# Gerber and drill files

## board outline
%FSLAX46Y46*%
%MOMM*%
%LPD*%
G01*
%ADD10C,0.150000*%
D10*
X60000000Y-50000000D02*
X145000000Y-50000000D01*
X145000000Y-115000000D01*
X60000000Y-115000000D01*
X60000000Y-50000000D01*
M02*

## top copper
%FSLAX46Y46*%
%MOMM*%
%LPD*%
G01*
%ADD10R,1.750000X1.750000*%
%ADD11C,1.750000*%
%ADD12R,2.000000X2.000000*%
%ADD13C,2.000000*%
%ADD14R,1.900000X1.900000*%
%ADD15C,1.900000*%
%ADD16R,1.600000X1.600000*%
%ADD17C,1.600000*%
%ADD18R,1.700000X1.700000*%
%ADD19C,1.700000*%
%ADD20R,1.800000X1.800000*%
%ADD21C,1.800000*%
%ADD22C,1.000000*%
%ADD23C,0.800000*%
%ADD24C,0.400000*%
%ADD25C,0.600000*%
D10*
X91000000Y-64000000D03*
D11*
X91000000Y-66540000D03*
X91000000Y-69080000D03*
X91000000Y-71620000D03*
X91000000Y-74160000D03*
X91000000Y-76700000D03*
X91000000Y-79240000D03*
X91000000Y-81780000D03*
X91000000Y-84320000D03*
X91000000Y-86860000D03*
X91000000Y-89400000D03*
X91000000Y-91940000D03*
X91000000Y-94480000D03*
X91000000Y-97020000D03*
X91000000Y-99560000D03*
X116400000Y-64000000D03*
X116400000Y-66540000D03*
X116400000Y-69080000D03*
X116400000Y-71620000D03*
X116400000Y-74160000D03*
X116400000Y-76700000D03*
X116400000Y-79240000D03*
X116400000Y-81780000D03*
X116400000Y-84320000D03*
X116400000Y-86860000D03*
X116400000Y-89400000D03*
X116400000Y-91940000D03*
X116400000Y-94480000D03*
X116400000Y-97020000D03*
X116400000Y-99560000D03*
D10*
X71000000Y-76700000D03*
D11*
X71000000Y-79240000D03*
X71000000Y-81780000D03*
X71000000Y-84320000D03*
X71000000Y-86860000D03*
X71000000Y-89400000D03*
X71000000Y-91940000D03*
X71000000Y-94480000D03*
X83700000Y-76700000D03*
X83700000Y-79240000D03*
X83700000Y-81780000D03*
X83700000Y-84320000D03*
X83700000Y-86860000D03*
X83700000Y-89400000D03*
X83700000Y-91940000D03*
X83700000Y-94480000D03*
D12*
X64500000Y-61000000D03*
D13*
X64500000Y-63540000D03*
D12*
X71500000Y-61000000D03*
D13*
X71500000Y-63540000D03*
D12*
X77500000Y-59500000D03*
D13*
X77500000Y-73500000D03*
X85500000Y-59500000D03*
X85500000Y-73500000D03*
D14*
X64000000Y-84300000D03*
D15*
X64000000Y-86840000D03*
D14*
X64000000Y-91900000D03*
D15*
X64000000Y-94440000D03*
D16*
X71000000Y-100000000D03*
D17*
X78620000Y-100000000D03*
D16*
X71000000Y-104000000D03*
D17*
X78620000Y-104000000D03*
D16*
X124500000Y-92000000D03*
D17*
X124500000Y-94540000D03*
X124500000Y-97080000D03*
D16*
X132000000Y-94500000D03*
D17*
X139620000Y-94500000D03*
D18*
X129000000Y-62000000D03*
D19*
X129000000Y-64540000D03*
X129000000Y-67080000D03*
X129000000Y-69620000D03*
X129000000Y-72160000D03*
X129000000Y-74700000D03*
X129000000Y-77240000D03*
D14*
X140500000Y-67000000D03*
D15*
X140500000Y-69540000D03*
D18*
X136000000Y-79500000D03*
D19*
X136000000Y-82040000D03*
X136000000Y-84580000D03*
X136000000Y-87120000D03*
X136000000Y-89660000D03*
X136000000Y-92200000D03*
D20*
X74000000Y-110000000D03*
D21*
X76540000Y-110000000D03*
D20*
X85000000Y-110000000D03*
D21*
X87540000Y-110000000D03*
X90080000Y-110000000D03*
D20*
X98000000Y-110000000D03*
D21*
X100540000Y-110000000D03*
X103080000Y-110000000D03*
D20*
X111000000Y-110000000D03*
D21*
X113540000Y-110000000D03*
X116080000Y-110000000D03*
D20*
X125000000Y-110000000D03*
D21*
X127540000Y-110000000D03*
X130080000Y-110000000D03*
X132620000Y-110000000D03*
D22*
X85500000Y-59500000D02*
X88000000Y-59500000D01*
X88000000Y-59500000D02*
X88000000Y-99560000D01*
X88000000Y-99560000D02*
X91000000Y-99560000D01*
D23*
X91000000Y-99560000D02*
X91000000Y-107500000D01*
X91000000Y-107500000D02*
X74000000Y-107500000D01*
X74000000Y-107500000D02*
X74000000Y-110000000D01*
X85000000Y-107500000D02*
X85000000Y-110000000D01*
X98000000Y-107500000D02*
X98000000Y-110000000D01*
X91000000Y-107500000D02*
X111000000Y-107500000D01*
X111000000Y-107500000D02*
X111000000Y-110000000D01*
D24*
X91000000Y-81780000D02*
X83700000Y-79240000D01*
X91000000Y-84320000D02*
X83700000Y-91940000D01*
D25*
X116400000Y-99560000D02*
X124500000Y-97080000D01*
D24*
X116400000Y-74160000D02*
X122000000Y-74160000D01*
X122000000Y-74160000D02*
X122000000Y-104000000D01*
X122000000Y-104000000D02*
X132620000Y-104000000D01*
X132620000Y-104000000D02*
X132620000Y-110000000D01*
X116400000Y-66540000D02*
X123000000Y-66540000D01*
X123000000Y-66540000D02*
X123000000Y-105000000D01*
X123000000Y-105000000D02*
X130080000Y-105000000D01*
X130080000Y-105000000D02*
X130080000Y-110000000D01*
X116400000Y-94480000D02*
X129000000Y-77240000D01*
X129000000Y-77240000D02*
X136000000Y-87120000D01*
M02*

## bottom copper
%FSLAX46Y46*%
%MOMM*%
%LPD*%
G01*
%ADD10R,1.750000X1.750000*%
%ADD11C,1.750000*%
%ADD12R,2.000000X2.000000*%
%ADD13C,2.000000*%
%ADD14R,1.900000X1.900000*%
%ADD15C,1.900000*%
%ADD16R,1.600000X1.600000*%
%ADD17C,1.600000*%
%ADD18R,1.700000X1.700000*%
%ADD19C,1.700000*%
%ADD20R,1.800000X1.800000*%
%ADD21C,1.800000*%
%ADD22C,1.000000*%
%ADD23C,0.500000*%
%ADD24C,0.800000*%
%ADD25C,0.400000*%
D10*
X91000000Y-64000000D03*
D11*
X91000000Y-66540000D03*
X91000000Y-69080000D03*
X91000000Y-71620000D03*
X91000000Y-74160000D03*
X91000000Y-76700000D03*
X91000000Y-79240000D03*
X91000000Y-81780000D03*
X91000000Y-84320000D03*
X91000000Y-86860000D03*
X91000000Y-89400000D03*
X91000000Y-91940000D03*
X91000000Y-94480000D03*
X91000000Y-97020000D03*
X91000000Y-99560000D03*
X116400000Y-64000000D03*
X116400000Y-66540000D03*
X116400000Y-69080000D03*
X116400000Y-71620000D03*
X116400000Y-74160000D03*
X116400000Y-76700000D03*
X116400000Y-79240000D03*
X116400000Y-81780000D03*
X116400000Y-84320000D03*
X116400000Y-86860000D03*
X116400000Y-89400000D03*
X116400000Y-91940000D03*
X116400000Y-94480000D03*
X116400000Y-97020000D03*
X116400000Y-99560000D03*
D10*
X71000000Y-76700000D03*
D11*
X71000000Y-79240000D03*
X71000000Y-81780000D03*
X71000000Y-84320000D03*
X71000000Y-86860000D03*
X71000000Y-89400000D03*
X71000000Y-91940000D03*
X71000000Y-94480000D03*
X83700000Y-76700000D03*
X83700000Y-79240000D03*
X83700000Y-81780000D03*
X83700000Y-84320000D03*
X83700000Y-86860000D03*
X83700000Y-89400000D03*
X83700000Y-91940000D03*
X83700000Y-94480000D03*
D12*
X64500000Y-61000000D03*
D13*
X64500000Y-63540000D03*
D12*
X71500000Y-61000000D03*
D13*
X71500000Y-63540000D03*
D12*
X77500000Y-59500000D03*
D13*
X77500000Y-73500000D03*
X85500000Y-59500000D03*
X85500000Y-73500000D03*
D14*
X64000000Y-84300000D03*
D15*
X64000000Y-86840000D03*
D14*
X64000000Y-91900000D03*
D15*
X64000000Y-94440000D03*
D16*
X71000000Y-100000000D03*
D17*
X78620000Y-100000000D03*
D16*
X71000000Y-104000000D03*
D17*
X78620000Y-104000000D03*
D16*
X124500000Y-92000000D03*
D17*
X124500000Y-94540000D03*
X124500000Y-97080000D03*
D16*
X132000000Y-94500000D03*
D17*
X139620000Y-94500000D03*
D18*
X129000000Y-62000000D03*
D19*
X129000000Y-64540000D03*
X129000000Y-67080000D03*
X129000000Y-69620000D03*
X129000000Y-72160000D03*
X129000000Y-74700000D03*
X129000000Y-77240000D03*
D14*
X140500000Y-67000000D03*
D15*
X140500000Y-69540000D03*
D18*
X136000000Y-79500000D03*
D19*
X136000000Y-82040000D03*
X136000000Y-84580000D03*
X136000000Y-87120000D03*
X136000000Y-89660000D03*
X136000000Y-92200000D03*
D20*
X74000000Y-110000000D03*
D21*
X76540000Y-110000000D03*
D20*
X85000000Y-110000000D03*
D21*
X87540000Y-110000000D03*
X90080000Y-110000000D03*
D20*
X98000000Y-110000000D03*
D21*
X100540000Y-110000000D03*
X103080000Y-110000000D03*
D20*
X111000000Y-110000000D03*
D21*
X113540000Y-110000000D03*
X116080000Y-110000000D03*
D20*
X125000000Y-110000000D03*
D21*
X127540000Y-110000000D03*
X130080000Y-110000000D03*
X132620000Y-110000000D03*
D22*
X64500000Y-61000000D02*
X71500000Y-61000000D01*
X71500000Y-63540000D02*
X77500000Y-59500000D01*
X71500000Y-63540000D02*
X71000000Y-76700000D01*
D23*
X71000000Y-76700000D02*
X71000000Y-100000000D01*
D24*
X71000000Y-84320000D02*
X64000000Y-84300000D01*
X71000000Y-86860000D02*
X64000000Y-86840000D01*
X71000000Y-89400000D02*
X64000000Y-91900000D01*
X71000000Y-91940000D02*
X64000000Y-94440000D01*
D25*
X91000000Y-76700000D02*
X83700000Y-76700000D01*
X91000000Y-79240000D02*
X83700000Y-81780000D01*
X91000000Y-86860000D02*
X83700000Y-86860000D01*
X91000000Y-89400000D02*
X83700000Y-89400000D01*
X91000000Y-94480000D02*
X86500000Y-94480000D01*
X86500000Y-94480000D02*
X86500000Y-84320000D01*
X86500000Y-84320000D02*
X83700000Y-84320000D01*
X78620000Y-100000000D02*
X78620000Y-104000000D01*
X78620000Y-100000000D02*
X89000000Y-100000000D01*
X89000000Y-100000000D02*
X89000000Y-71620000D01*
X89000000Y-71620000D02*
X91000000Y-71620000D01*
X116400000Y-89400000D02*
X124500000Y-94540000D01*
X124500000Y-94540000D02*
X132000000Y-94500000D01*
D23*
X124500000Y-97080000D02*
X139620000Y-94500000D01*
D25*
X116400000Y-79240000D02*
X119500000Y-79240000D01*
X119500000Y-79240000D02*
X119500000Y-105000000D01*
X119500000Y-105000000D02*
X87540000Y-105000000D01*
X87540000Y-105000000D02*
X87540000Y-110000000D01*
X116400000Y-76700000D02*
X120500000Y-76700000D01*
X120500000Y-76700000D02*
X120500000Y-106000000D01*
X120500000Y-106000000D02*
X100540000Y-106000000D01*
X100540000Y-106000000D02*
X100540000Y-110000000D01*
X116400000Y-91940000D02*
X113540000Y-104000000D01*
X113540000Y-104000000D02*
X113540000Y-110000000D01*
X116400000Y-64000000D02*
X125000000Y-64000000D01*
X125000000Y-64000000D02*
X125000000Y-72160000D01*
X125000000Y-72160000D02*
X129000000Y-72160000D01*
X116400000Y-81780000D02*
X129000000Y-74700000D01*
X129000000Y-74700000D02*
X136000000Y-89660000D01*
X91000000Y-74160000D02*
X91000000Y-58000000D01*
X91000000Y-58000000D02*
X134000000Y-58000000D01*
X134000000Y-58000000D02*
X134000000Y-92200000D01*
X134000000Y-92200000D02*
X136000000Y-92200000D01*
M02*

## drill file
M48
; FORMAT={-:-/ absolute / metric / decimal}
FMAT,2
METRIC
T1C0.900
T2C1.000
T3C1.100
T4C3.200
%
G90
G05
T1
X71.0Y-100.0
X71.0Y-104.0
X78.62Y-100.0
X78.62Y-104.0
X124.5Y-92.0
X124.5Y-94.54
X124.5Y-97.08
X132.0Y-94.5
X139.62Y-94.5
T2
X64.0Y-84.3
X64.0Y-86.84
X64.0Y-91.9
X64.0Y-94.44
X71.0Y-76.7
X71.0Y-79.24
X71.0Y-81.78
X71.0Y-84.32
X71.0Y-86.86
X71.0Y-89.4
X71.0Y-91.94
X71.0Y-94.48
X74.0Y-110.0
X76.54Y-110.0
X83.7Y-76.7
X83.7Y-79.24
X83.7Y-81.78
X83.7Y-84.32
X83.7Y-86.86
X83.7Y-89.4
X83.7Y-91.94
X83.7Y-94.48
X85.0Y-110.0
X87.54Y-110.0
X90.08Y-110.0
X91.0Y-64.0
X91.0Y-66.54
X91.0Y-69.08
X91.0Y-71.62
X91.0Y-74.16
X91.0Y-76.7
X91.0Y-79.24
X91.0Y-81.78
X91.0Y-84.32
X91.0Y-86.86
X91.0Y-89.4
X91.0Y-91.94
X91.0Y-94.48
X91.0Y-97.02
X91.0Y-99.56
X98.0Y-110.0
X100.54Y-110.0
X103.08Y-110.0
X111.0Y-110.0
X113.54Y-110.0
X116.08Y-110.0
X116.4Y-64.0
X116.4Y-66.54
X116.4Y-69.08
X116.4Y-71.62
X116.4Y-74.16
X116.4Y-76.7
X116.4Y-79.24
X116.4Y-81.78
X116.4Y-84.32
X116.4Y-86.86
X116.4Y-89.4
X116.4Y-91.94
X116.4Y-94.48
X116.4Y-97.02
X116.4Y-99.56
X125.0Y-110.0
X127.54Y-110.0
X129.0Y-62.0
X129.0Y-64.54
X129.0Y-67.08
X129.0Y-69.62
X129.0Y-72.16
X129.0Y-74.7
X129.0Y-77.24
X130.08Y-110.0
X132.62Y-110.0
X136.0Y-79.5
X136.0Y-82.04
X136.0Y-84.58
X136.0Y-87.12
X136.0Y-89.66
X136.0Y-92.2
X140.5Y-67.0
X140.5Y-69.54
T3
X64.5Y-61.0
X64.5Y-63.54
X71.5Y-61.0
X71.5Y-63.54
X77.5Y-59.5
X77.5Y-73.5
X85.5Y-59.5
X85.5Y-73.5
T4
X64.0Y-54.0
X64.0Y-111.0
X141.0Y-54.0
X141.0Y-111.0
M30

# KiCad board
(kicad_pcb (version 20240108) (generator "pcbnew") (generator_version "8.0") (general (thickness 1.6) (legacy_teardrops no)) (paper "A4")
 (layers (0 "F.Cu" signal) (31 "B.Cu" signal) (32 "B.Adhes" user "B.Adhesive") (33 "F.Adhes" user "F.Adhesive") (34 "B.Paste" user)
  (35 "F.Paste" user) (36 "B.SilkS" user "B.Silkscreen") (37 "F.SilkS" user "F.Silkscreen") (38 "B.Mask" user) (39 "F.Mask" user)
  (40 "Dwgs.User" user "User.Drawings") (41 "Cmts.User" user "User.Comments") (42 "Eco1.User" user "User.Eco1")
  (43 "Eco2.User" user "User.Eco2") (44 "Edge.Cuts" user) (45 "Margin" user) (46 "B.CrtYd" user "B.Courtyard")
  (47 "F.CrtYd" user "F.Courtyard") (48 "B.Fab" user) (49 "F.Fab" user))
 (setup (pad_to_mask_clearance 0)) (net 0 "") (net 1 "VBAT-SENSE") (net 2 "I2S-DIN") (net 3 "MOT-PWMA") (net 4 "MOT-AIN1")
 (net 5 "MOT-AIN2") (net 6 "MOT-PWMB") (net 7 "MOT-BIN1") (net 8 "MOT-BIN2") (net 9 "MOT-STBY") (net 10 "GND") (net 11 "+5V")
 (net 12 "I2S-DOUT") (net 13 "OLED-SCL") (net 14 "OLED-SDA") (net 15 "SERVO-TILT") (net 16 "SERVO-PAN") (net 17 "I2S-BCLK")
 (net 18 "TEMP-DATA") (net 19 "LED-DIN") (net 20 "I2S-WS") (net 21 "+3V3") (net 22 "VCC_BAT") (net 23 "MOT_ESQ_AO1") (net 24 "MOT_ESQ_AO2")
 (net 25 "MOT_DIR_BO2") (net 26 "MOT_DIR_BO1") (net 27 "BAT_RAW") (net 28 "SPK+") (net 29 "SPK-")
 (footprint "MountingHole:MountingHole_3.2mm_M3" (layer "F.Cu") (at 64.0 54.0 0)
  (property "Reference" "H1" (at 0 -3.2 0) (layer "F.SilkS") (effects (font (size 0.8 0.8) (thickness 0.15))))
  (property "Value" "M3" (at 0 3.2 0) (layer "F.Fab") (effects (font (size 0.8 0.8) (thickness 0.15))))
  (pad "1" np_thru_hole circle (at 0 0) (size 3.2 3.2) (drill 3.2) (layers "*.Cu" "*.Mask")))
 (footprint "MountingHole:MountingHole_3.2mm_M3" (layer "F.Cu") (at 141.0 54.0 0)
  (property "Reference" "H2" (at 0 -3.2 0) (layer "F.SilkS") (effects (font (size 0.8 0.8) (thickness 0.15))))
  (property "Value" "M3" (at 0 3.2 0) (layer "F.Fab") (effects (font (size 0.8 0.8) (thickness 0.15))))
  (pad "1" np_thru_hole circle (at 0 0) (size 3.2 3.2) (drill 3.2) (layers "*.Cu" "*.Mask")))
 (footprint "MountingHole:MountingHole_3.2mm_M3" (layer "F.Cu") (at 64.0 111.0 0)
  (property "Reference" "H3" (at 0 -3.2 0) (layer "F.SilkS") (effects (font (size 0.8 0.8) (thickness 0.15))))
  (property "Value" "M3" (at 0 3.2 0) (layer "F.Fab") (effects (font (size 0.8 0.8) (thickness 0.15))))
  (pad "1" np_thru_hole circle (at 0 0) (size 3.2 3.2) (drill 3.2) (layers "*.Cu" "*.Mask")))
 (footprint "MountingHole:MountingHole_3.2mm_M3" (layer "F.Cu") (at 141.0 111.0 0)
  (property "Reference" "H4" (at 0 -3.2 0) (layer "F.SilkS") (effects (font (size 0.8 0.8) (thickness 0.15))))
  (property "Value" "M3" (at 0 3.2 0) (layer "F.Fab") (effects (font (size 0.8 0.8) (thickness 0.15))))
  (pad "1" np_thru_hole circle (at 0 0) (size 3.2 3.2) (drill 3.2) (layers "*.Cu" "*.Mask")))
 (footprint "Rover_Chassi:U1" (layer "F.Cu") (at 91.0 64.0 0)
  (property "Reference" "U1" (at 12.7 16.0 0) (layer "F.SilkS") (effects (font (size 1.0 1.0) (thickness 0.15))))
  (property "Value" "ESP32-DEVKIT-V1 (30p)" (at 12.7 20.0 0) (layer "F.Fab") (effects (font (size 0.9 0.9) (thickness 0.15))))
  (pad "1" thru_hole rect (at 0.0 0.0) (size 1.75 1.75) (drill 1.0) (layers "*.Cu" "*.Mask"))
  (pad "2" thru_hole circle (at 0.0 2.54) (size 1.75 1.75) (drill 1.0) (layers "*.Cu" "*.Mask"))
  (pad "3" thru_hole circle (at 0.0 5.08) (size 1.75 1.75) (drill 1.0) (layers "*.Cu" "*.Mask"))
  (pad "4" thru_hole circle (at 0.0 7.62) (size 1.75 1.75) (drill 1.0) (layers "*.Cu" "*.Mask") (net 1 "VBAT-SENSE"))
  (pad "5" thru_hole circle (at 0.0 10.16) (size 1.75 1.75) (drill 1.0) (layers "*.Cu" "*.Mask") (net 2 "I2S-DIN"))
  (pad "6" thru_hole circle (at 0.0 12.7) (size 1.75 1.75) (drill 1.0) (layers "*.Cu" "*.Mask") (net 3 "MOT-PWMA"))
  (pad "7" thru_hole circle (at 0.0 15.24) (size 1.75 1.75) (drill 1.0) (layers "*.Cu" "*.Mask") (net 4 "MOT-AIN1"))
  (pad "8" thru_hole circle (at 0.0 17.78) (size 1.75 1.75) (drill 1.0) (layers "*.Cu" "*.Mask") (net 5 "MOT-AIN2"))
  (pad "9" thru_hole circle (at 0.0 20.32) (size 1.75 1.75) (drill 1.0) (layers "*.Cu" "*.Mask") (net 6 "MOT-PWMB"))
  (pad "10" thru_hole circle (at 0.0 22.86) (size 1.75 1.75) (drill 1.0) (layers "*.Cu" "*.Mask") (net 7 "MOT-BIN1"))
  (pad "11" thru_hole circle (at 0.0 25.4) (size 1.75 1.75) (drill 1.0) (layers "*.Cu" "*.Mask") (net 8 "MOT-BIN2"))
  (pad "12" thru_hole circle (at 0.0 27.94) (size 1.75 1.75) (drill 1.0) (layers "*.Cu" "*.Mask"))
  (pad "13" thru_hole circle (at 0.0 30.48) (size 1.75 1.75) (drill 1.0) (layers "*.Cu" "*.Mask") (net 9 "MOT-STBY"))
  (pad "14" thru_hole circle (at 0.0 33.02) (size 1.75 1.75) (drill 1.0) (layers "*.Cu" "*.Mask") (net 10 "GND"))
  (pad "15" thru_hole circle (at 0.0 35.56) (size 1.75 1.75) (drill 1.0) (layers "*.Cu" "*.Mask") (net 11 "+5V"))
  (pad "16" thru_hole circle (at 25.4 0.0) (size 1.75 1.75) (drill 1.0) (layers "*.Cu" "*.Mask") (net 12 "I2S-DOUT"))
  (pad "17" thru_hole circle (at 25.4 2.54) (size 1.75 1.75) (drill 1.0) (layers "*.Cu" "*.Mask") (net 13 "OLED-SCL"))
  (pad "18" thru_hole circle (at 25.4 5.08) (size 1.75 1.75) (drill 1.0) (layers "*.Cu" "*.Mask"))
  (pad "19" thru_hole circle (at 25.4 7.62) (size 1.75 1.75) (drill 1.0) (layers "*.Cu" "*.Mask"))
  (pad "20" thru_hole circle (at 25.4 10.16) (size 1.75 1.75) (drill 1.0) (layers "*.Cu" "*.Mask") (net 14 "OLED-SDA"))
  (pad "21" thru_hole circle (at 25.4 12.7) (size 1.75 1.75) (drill 1.0) (layers "*.Cu" "*.Mask") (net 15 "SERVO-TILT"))
  (pad "22" thru_hole circle (at 25.4 15.24) (size 1.75 1.75) (drill 1.0) (layers "*.Cu" "*.Mask") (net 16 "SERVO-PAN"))
  (pad "23" thru_hole circle (at 25.4 17.78) (size 1.75 1.75) (drill 1.0) (layers "*.Cu" "*.Mask") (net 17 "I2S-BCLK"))
  (pad "24" thru_hole circle (at 25.4 20.32) (size 1.75 1.75) (drill 1.0) (layers "*.Cu" "*.Mask"))
  (pad "25" thru_hole circle (at 25.4 22.86) (size 1.75 1.75) (drill 1.0) (layers "*.Cu" "*.Mask"))
  (pad "26" thru_hole circle (at 25.4 25.4) (size 1.75 1.75) (drill 1.0) (layers "*.Cu" "*.Mask") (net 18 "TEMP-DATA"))
  (pad "27" thru_hole circle (at 25.4 27.94) (size 1.75 1.75) (drill 1.0) (layers "*.Cu" "*.Mask") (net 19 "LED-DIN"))
  (pad "28" thru_hole circle (at 25.4 30.48) (size 1.75 1.75) (drill 1.0) (layers "*.Cu" "*.Mask") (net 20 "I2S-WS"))
  (pad "29" thru_hole circle (at 25.4 33.02) (size 1.75 1.75) (drill 1.0) (layers "*.Cu" "*.Mask") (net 10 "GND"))
  (pad "30" thru_hole circle (at 25.4 35.56) (size 1.75 1.75) (drill 1.0) (layers "*.Cu" "*.Mask") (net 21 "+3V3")))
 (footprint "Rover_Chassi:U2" (layer "F.Cu") (at 71.0 76.7 0)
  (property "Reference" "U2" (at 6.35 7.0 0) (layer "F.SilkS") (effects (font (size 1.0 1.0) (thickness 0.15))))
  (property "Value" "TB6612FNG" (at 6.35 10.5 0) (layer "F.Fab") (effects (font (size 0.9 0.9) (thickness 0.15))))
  (pad "1" thru_hole rect (at 0.0 0.0) (size 1.75 1.75) (drill 1.0) (layers "*.Cu" "*.Mask") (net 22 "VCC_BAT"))
  (pad "2" thru_hole circle (at 0.0 2.54) (size 1.75 1.75) (drill 1.0) (layers "*.Cu" "*.Mask") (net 21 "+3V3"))
  (pad "3" thru_hole circle (at 0.0 5.08) (size 1.75 1.75) (drill 1.0) (layers "*.Cu" "*.Mask") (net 10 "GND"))
  (pad "4" thru_hole circle (at 0.0 7.62) (size 1.75 1.75) (drill 1.0) (layers "*.Cu" "*.Mask") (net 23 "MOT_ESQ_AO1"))
  (pad "5" thru_hole circle (at 0.0 10.16) (size 1.75 1.75) (drill 1.0) (layers "*.Cu" "*.Mask") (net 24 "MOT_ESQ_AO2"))
  (pad "6" thru_hole circle (at 0.0 12.7) (size 1.75 1.75) (drill 1.0) (layers "*.Cu" "*.Mask") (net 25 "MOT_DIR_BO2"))
  (pad "7" thru_hole circle (at 0.0 15.24) (size 1.75 1.75) (drill 1.0) (layers "*.Cu" "*.Mask") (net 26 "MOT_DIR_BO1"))
  (pad "8" thru_hole circle (at 0.0 17.78) (size 1.75 1.75) (drill 1.0) (layers "*.Cu" "*.Mask") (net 10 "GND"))
  (pad "9" thru_hole circle (at 12.7 0.0) (size 1.75 1.75) (drill 1.0) (layers "*.Cu" "*.Mask") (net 3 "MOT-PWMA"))
  (pad "10" thru_hole circle (at 12.7 2.54) (size 1.75 1.75) (drill 1.0) (layers "*.Cu" "*.Mask") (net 5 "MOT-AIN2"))
  (pad "11" thru_hole circle (at 12.7 5.08) (size 1.75 1.75) (drill 1.0) (layers "*.Cu" "*.Mask") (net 4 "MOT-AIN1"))
  (pad "12" thru_hole circle (at 12.7 7.62) (size 1.75 1.75) (drill 1.0) (layers "*.Cu" "*.Mask") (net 9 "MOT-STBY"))
  (pad "13" thru_hole circle (at 12.7 10.16) (size 1.75 1.75) (drill 1.0) (layers "*.Cu" "*.Mask") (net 7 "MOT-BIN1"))
  (pad "14" thru_hole circle (at 12.7 12.7) (size 1.75 1.75) (drill 1.0) (layers "*.Cu" "*.Mask") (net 8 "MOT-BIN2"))
  (pad "15" thru_hole circle (at 12.7 15.24) (size 1.75 1.75) (drill 1.0) (layers "*.Cu" "*.Mask") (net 6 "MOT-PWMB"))
  (pad "16" thru_hole circle (at 12.7 17.78) (size 1.75 1.75) (drill 1.0) (layers "*.Cu" "*.Mask") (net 10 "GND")))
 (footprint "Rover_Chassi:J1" (layer "F.Cu") (at 64.5 61.0 0)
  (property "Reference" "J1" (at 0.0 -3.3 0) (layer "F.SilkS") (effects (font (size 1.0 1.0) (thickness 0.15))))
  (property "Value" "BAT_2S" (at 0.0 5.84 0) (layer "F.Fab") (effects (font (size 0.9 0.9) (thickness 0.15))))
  (pad "1" thru_hole rect (at 0.0 0.0) (size 2.0 2.0) (drill 1.1) (layers "*.Cu" "*.Mask") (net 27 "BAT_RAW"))
  (pad "2" thru_hole circle (at 0.0 2.54) (size 2.0 2.0) (drill 1.1) (layers "*.Cu" "*.Mask") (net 10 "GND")))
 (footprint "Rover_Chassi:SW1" (layer "F.Cu") (at 71.5 61.0 0)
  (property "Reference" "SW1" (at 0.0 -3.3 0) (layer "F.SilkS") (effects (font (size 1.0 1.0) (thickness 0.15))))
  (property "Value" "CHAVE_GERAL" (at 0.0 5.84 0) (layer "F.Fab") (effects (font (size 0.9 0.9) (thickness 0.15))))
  (pad "1" thru_hole rect (at 0.0 0.0) (size 2.0 2.0) (drill 1.1) (layers "*.Cu" "*.Mask") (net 27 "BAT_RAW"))
  (pad "2" thru_hole circle (at 0.0 2.54) (size 2.0 2.0) (drill 1.1) (layers "*.Cu" "*.Mask") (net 22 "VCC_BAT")))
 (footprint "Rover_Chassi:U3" (layer "F.Cu") (at 77.5 59.5 0)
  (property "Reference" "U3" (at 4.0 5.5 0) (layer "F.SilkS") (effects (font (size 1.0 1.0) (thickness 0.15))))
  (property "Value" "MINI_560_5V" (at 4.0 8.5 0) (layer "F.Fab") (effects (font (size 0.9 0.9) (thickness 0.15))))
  (pad "1" thru_hole rect (at 0.0 0.0) (size 2.0 2.0) (drill 1.1) (layers "*.Cu" "*.Mask") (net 22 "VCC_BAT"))
  (pad "2" thru_hole circle (at 0.0 14.0) (size 2.0 2.0) (drill 1.1) (layers "*.Cu" "*.Mask") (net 10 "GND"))
  (pad "3" thru_hole circle (at 8.0 0.0) (size 2.0 2.0) (drill 1.1) (layers "*.Cu" "*.Mask") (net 11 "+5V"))
  (pad "4" thru_hole circle (at 8.0 14.0) (size 2.0 2.0) (drill 1.1) (layers "*.Cu" "*.Mask") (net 10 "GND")))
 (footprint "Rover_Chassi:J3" (layer "F.Cu") (at 64.0 84.3 0)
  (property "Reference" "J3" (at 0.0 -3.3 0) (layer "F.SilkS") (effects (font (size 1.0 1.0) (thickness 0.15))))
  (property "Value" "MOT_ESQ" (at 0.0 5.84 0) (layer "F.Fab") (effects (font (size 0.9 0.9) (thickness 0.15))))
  (pad "1" thru_hole rect (at 0.0 0.0) (size 1.9 1.9) (drill 1.0) (layers "*.Cu" "*.Mask") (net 23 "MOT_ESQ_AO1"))
  (pad "2" thru_hole circle (at 0.0 2.54) (size 1.9 1.9) (drill 1.0) (layers "*.Cu" "*.Mask") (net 24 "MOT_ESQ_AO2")))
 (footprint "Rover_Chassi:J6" (layer "F.Cu") (at 64.0 91.9 0)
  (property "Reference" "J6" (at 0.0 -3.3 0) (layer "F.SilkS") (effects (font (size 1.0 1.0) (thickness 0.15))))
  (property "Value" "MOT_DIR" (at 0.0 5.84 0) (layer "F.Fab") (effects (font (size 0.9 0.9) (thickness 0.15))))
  (pad "1" thru_hole rect (at 0.0 0.0) (size 1.9 1.9) (drill 1.0) (layers "*.Cu" "*.Mask") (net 25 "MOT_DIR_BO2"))
  (pad "2" thru_hole circle (at 0.0 2.54) (size 1.9 1.9) (drill 1.0) (layers "*.Cu" "*.Mask") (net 26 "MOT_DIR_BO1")))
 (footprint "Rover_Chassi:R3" (layer "F.Cu") (at 71.0 100.0 0)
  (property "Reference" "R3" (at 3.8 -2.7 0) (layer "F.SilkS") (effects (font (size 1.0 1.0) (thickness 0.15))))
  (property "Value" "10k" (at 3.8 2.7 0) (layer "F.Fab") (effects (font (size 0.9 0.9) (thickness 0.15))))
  (pad "1" thru_hole rect (at 0.0 0.0) (size 1.6 1.6) (drill 0.9) (layers "*.Cu" "*.Mask") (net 22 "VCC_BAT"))
  (pad "2" thru_hole circle (at 7.62 0.0) (size 1.6 1.6) (drill 0.9) (layers "*.Cu" "*.Mask") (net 1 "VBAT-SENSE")))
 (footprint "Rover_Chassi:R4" (layer "F.Cu") (at 71.0 104.0 0)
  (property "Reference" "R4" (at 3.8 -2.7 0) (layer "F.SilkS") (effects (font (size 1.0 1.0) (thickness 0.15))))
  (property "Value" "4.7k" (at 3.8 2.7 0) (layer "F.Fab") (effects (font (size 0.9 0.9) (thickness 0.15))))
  (pad "1" thru_hole rect (at 0.0 0.0) (size 1.6 1.6) (drill 0.9) (layers "*.Cu" "*.Mask") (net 10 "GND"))
  (pad "2" thru_hole circle (at 7.62 0.0) (size 1.6 1.6) (drill 0.9) (layers "*.Cu" "*.Mask") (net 1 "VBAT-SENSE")))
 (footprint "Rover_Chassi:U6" (layer "F.Cu") (at 124.5 92.0 0)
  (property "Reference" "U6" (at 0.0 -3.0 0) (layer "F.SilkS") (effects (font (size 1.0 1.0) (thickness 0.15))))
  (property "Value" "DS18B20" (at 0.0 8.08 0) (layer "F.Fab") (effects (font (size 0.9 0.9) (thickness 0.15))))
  (pad "1" thru_hole rect (at 0.0 0.0) (size 1.6 1.6) (drill 0.9) (layers "*.Cu" "*.Mask") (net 10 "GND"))
  (pad "2" thru_hole circle (at 0.0 2.54) (size 1.6 1.6) (drill 0.9) (layers "*.Cu" "*.Mask") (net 18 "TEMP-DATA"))
  (pad "3" thru_hole circle (at 0.0 5.08) (size 1.6 1.6) (drill 0.9) (layers "*.Cu" "*.Mask") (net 21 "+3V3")))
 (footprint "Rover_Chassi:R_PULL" (layer "F.Cu") (at 132.0 94.5 0)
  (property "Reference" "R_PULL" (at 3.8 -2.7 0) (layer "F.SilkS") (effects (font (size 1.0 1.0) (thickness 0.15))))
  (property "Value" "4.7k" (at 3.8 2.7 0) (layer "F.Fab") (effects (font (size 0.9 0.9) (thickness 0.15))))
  (pad "1" thru_hole rect (at 0.0 0.0) (size 1.6 1.6) (drill 0.9) (layers "*.Cu" "*.Mask") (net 18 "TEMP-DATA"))
  (pad "2" thru_hole circle (at 7.62 0.0) (size 1.6 1.6) (drill 0.9) (layers "*.Cu" "*.Mask") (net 21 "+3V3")))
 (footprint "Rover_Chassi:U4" (layer "F.Cu") (at 129.0 62.0 0)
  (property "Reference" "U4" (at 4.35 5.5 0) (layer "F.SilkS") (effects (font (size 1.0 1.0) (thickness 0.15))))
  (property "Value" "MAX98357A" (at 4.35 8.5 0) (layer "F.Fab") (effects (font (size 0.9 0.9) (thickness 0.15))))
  (pad "1" thru_hole rect (at 0.0 0.0) (size 1.7 1.7) (drill 1.0) (layers "*.Cu" "*.Mask") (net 11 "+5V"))
  (pad "2" thru_hole circle (at 0.0 2.54) (size 1.7 1.7) (drill 1.0) (layers "*.Cu" "*.Mask") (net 10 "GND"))
  (pad "3" thru_hole circle (at 0.0 5.08) (size 1.7 1.7) (drill 1.0) (layers "*.Cu" "*.Mask"))
  (pad "4" thru_hole circle (at 0.0 7.62) (size 1.7 1.7) (drill 1.0) (layers "*.Cu" "*.Mask"))
  (pad "5" thru_hole circle (at 0.0 10.16) (size 1.7 1.7) (drill 1.0) (layers "*.Cu" "*.Mask") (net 12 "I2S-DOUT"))
  (pad "6" thru_hole circle (at 0.0 12.7) (size 1.7 1.7) (drill 1.0) (layers "*.Cu" "*.Mask") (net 17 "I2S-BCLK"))
  (pad "7" thru_hole circle (at 0.0 15.24) (size 1.7 1.7) (drill 1.0) (layers "*.Cu" "*.Mask") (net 20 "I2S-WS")))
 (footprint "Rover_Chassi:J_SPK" (layer "F.Cu") (at 140.5 67.0 0)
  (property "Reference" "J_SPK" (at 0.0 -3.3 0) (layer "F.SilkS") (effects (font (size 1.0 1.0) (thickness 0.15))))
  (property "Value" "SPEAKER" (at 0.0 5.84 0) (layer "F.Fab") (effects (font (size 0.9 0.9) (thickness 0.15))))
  (pad "1" thru_hole rect (at 0.0 0.0) (size 1.9 1.9) (drill 1.0) (layers "*.Cu" "*.Mask") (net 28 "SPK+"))
  (pad "2" thru_hole circle (at 0.0 2.54) (size 1.9 1.9) (drill 1.0) (layers "*.Cu" "*.Mask") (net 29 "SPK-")))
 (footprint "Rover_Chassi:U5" (layer "F.Cu") (at 136.0 79.5 0)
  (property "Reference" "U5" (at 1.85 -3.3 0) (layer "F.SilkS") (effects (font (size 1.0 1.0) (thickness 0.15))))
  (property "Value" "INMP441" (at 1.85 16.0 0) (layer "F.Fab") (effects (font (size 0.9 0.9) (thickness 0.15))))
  (pad "1" thru_hole rect (at 0.0 0.0) (size 1.7 1.7) (drill 1.0) (layers "*.Cu" "*.Mask") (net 21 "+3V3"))
  (pad "2" thru_hole circle (at 0.0 2.54) (size 1.7 1.7) (drill 1.0) (layers "*.Cu" "*.Mask") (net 10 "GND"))
  (pad "3" thru_hole circle (at 0.0 5.08) (size 1.7 1.7) (drill 1.0) (layers "*.Cu" "*.Mask") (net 10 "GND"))
  (pad "4" thru_hole circle (at 0.0 7.62) (size 1.7 1.7) (drill 1.0) (layers "*.Cu" "*.Mask") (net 20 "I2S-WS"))
  (pad "5" thru_hole circle (at 0.0 10.16) (size 1.7 1.7) (drill 1.0) (layers "*.Cu" "*.Mask") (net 17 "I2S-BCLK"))
  (pad "6" thru_hole circle (at 0.0 12.7) (size 1.7 1.7) (drill 1.0) (layers "*.Cu" "*.Mask") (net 2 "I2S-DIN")))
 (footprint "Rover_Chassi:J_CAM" (layer "F.Cu") (at 74.0 110.0 0)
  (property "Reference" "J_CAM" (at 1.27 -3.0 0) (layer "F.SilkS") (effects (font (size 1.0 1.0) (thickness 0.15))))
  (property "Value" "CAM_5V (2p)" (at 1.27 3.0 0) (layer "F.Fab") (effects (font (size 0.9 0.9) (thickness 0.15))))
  (pad "1" thru_hole rect (at 0.0 0.0) (size 1.8 1.8) (drill 1.0) (layers "*.Cu" "*.Mask") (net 11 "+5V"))
  (pad "2" thru_hole circle (at 2.54 0.0) (size 1.8 1.8) (drill 1.0) (layers "*.Cu" "*.Mask") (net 10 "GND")))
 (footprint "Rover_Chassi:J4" (layer "F.Cu") (at 85.0 110.0 0)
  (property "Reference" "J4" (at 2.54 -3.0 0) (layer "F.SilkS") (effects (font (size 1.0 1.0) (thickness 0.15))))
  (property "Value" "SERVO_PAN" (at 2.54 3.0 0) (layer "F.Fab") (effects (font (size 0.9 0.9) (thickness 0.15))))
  (pad "1" thru_hole rect (at 0.0 0.0) (size 1.8 1.8) (drill 1.0) (layers "*.Cu" "*.Mask") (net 11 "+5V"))
  (pad "2" thru_hole circle (at 2.54 0.0) (size 1.8 1.8) (drill 1.0) (layers "*.Cu" "*.Mask") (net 16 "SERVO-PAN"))
  (pad "3" thru_hole circle (at 5.08 0.0) (size 1.8 1.8) (drill 1.0) (layers "*.Cu" "*.Mask") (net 10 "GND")))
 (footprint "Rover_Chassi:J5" (layer "F.Cu") (at 98.0 110.0 0)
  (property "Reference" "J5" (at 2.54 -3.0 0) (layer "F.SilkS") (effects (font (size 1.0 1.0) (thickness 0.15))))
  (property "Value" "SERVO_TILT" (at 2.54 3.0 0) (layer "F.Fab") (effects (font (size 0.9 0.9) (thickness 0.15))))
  (pad "1" thru_hole rect (at 0.0 0.0) (size 1.8 1.8) (drill 1.0) (layers "*.Cu" "*.Mask") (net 11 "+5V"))
  (pad "2" thru_hole circle (at 2.54 0.0) (size 1.8 1.8) (drill 1.0) (layers "*.Cu" "*.Mask") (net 15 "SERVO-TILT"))
  (pad "3" thru_hole circle (at 5.08 0.0) (size 1.8 1.8) (drill 1.0) (layers "*.Cu" "*.Mask") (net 10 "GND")))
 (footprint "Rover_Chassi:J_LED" (layer "F.Cu") (at 111.0 110.0 0)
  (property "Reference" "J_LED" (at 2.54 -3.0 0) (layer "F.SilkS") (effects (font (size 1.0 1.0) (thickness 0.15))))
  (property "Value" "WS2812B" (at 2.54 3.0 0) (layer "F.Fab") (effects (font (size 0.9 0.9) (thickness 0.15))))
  (pad "1" thru_hole rect (at 0.0 0.0) (size 1.8 1.8) (drill 1.0) (layers "*.Cu" "*.Mask") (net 11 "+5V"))
  (pad "2" thru_hole circle (at 2.54 0.0) (size 1.8 1.8) (drill 1.0) (layers "*.Cu" "*.Mask") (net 19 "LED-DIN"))
  (pad "3" thru_hole circle (at 5.08 0.0) (size 1.8 1.8) (drill 1.0) (layers "*.Cu" "*.Mask") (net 10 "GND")))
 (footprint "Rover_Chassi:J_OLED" (layer "F.Cu") (at 125.0 110.0 0)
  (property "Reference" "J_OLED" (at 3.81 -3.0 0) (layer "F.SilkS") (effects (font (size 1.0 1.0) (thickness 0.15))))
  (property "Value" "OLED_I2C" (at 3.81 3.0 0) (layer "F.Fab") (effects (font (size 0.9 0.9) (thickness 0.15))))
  (pad "1" thru_hole rect (at 0.0 0.0) (size 1.8 1.8) (drill 1.0) (layers "*.Cu" "*.Mask") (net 10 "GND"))
  (pad "2" thru_hole circle (at 2.54 0.0) (size 1.8 1.8) (drill 1.0) (layers "*.Cu" "*.Mask") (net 21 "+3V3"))
  (pad "3" thru_hole circle (at 5.08 0.0) (size 1.8 1.8) (drill 1.0) (layers "*.Cu" "*.Mask") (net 13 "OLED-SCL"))
  (pad "4" thru_hole circle (at 7.62 0.0) (size 1.8 1.8) (drill 1.0) (layers "*.Cu" "*.Mask") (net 14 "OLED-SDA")))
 (gr_rect (start 60.0 50.0) (end 145.0 115.0) (stroke (width 0.15) (type default)) (fill no) (layer "Edge.Cuts"))
 (segment (start 64.5 61.0) (end 71.5 61.0) (width 1.0) (layer "B.Cu") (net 27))
 (segment (start 71.5 63.54) (end 77.5 59.5) (width 1.0) (layer "B.Cu") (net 22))
 (segment (start 71.5 63.54) (end 71.0 76.7) (width 1.0) (layer "B.Cu") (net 22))
 (segment (start 71.0 76.7) (end 71.0 100.0) (width 0.5) (layer "B.Cu") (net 22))
 (segment (start 85.5 59.5) (end 88.0 59.5) (width 1.0) (layer "F.Cu") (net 11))
 (segment (start 88.0 59.5) (end 88.0 99.56) (width 1.0) (layer "F.Cu") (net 11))
 (segment (start 88.0 99.56) (end 91.0 99.56) (width 1.0) (layer "F.Cu") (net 11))
 (segment (start 91.0 99.56) (end 91.0 107.5) (width 0.8) (layer "F.Cu") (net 11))
 (segment (start 91.0 107.5) (end 74.0 107.5) (width 0.8) (layer "F.Cu") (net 11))
 (segment (start 74.0 107.5) (end 74.0 110.0) (width 0.8) (layer "F.Cu") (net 11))
 (segment (start 85.0 107.5) (end 85.0 110.0) (width 0.8) (layer "F.Cu") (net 11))
 (segment (start 98.0 107.5) (end 98.0 110.0) (width 0.8) (layer "F.Cu") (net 11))
 (segment (start 91.0 107.5) (end 111.0 107.5) (width 0.8) (layer "F.Cu") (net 11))
 (segment (start 111.0 107.5) (end 111.0 110.0) (width 0.8) (layer "F.Cu") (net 11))
 (segment (start 71.0 84.32) (end 64.0 84.3) (width 0.8) (layer "B.Cu") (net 23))
 (segment (start 71.0 86.86) (end 64.0 86.84) (width 0.8) (layer "B.Cu") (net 24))
 (segment (start 71.0 89.4) (end 64.0 91.9) (width 0.8) (layer "B.Cu") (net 25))
 (segment (start 71.0 91.94) (end 64.0 94.44) (width 0.8) (layer "B.Cu") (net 26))
 (segment (start 91.0 76.7) (end 83.7 76.7) (width 0.4) (layer "B.Cu") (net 3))
 (segment (start 91.0 79.24) (end 83.7 81.78) (width 0.4) (layer "B.Cu") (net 4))
 (segment (start 91.0 81.78) (end 83.7 79.24) (width 0.4) (layer "F.Cu") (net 5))
 (segment (start 91.0 84.32) (end 83.7 91.94) (width 0.4) (layer "F.Cu") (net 6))
 (segment (start 91.0 86.86) (end 83.7 86.86) (width 0.4) (layer "B.Cu") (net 7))
 (segment (start 91.0 89.4) (end 83.7 89.4) (width 0.4) (layer "B.Cu") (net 8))
 (segment (start 91.0 94.48) (end 86.5 94.48) (width 0.4) (layer "B.Cu") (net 9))
 (segment (start 86.5 94.48) (end 86.5 84.32) (width 0.4) (layer "B.Cu") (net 9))
 (segment (start 86.5 84.32) (end 83.7 84.32) (width 0.4) (layer "B.Cu") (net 9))
 (segment (start 78.62 100.0) (end 78.62 104.0) (width 0.4) (layer "B.Cu") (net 1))
 (segment (start 78.62 100.0) (end 89.0 100.0) (width 0.4) (layer "B.Cu") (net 1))
 (segment (start 89.0 100.0) (end 89.0 71.62) (width 0.4) (layer "B.Cu") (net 1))
 (segment (start 89.0 71.62) (end 91.0 71.62) (width 0.4) (layer "B.Cu") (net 1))
 (segment (start 116.4 89.4) (end 124.5 94.54) (width 0.4) (layer "B.Cu") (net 18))
 (segment (start 124.5 94.54) (end 132.0 94.5) (width 0.4) (layer "B.Cu") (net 18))
 (segment (start 124.5 97.08) (end 139.62 94.5) (width 0.5) (layer "B.Cu") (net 21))
 (segment (start 116.4 99.56) (end 124.5 97.08) (width 0.6) (layer "F.Cu") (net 21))
 (segment (start 116.4 79.24) (end 119.5 79.24) (width 0.4) (layer "B.Cu") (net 16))
 (segment (start 119.5 79.24) (end 119.5 105.0) (width 0.4) (layer "B.Cu") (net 16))
 (segment (start 119.5 105.0) (end 87.54 105.0) (width 0.4) (layer "B.Cu") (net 16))
 (segment (start 87.54 105.0) (end 87.54 110.0) (width 0.4) (layer "B.Cu") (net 16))
 (segment (start 116.4 76.7) (end 120.5 76.7) (width 0.4) (layer "B.Cu") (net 15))
 (segment (start 120.5 76.7) (end 120.5 106.0) (width 0.4) (layer "B.Cu") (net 15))
 (segment (start 120.5 106.0) (end 100.54 106.0) (width 0.4) (layer "B.Cu") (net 15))
 (segment (start 100.54 106.0) (end 100.54 110.0) (width 0.4) (layer "B.Cu") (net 15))
 (segment (start 116.4 91.94) (end 113.54 104.0) (width 0.4) (layer "B.Cu") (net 19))
 (segment (start 113.54 104.0) (end 113.54 110.0) (width 0.4) (layer "B.Cu") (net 19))
 (segment (start 116.4 74.16) (end 122.0 74.16) (width 0.4) (layer "F.Cu") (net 14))
 (segment (start 122.0 74.16) (end 122.0 104.0) (width 0.4) (layer "F.Cu") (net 14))
 (segment (start 122.0 104.0) (end 132.62 104.0) (width 0.4) (layer "F.Cu") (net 14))
 (segment (start 132.62 104.0) (end 132.62 110.0) (width 0.4) (layer "F.Cu") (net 14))
 (segment (start 116.4 66.54) (end 123.0 66.54) (width 0.4) (layer "F.Cu") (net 13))
 (segment (start 123.0 66.54) (end 123.0 105.0) (width 0.4) (layer "F.Cu") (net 13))
 (segment (start 123.0 105.0) (end 130.08 105.0) (width 0.4) (layer "F.Cu") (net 13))
 (segment (start 130.08 105.0) (end 130.08 110.0) (width 0.4) (layer "F.Cu") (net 13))
 (segment (start 116.4 64.0) (end 125.0 64.0) (width 0.4) (layer "B.Cu") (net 12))
 (segment (start 125.0 64.0) (end 125.0 72.16) (width 0.4) (layer "B.Cu") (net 12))
 (segment (start 125.0 72.16) (end 129.0 72.16) (width 0.4) (layer "B.Cu") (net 12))
 (segment (start 116.4 81.78) (end 129.0 74.7) (width 0.4) (layer "B.Cu") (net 17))
 (segment (start 129.0 74.7) (end 136.0 89.66) (width 0.4) (layer "B.Cu") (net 17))
 (segment (start 116.4 94.48) (end 129.0 77.24) (width 0.4) (layer "F.Cu") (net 20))
 (segment (start 129.0 77.24) (end 136.0 87.12) (width 0.4) (layer "F.Cu") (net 20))
 (segment (start 91.0 74.16) (end 91.0 58.0) (width 0.4) (layer "B.Cu") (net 2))
 (segment (start 91.0 58.0) (end 134.0 58.0) (width 0.4) (layer "B.Cu") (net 2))
 (segment (start 134.0 58.0) (end 134.0 92.2) (width 0.4) (layer "B.Cu") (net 2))
 (segment (start 134.0 92.2) (end 136.0 92.2) (width 0.4) (layer "B.Cu") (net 2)))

